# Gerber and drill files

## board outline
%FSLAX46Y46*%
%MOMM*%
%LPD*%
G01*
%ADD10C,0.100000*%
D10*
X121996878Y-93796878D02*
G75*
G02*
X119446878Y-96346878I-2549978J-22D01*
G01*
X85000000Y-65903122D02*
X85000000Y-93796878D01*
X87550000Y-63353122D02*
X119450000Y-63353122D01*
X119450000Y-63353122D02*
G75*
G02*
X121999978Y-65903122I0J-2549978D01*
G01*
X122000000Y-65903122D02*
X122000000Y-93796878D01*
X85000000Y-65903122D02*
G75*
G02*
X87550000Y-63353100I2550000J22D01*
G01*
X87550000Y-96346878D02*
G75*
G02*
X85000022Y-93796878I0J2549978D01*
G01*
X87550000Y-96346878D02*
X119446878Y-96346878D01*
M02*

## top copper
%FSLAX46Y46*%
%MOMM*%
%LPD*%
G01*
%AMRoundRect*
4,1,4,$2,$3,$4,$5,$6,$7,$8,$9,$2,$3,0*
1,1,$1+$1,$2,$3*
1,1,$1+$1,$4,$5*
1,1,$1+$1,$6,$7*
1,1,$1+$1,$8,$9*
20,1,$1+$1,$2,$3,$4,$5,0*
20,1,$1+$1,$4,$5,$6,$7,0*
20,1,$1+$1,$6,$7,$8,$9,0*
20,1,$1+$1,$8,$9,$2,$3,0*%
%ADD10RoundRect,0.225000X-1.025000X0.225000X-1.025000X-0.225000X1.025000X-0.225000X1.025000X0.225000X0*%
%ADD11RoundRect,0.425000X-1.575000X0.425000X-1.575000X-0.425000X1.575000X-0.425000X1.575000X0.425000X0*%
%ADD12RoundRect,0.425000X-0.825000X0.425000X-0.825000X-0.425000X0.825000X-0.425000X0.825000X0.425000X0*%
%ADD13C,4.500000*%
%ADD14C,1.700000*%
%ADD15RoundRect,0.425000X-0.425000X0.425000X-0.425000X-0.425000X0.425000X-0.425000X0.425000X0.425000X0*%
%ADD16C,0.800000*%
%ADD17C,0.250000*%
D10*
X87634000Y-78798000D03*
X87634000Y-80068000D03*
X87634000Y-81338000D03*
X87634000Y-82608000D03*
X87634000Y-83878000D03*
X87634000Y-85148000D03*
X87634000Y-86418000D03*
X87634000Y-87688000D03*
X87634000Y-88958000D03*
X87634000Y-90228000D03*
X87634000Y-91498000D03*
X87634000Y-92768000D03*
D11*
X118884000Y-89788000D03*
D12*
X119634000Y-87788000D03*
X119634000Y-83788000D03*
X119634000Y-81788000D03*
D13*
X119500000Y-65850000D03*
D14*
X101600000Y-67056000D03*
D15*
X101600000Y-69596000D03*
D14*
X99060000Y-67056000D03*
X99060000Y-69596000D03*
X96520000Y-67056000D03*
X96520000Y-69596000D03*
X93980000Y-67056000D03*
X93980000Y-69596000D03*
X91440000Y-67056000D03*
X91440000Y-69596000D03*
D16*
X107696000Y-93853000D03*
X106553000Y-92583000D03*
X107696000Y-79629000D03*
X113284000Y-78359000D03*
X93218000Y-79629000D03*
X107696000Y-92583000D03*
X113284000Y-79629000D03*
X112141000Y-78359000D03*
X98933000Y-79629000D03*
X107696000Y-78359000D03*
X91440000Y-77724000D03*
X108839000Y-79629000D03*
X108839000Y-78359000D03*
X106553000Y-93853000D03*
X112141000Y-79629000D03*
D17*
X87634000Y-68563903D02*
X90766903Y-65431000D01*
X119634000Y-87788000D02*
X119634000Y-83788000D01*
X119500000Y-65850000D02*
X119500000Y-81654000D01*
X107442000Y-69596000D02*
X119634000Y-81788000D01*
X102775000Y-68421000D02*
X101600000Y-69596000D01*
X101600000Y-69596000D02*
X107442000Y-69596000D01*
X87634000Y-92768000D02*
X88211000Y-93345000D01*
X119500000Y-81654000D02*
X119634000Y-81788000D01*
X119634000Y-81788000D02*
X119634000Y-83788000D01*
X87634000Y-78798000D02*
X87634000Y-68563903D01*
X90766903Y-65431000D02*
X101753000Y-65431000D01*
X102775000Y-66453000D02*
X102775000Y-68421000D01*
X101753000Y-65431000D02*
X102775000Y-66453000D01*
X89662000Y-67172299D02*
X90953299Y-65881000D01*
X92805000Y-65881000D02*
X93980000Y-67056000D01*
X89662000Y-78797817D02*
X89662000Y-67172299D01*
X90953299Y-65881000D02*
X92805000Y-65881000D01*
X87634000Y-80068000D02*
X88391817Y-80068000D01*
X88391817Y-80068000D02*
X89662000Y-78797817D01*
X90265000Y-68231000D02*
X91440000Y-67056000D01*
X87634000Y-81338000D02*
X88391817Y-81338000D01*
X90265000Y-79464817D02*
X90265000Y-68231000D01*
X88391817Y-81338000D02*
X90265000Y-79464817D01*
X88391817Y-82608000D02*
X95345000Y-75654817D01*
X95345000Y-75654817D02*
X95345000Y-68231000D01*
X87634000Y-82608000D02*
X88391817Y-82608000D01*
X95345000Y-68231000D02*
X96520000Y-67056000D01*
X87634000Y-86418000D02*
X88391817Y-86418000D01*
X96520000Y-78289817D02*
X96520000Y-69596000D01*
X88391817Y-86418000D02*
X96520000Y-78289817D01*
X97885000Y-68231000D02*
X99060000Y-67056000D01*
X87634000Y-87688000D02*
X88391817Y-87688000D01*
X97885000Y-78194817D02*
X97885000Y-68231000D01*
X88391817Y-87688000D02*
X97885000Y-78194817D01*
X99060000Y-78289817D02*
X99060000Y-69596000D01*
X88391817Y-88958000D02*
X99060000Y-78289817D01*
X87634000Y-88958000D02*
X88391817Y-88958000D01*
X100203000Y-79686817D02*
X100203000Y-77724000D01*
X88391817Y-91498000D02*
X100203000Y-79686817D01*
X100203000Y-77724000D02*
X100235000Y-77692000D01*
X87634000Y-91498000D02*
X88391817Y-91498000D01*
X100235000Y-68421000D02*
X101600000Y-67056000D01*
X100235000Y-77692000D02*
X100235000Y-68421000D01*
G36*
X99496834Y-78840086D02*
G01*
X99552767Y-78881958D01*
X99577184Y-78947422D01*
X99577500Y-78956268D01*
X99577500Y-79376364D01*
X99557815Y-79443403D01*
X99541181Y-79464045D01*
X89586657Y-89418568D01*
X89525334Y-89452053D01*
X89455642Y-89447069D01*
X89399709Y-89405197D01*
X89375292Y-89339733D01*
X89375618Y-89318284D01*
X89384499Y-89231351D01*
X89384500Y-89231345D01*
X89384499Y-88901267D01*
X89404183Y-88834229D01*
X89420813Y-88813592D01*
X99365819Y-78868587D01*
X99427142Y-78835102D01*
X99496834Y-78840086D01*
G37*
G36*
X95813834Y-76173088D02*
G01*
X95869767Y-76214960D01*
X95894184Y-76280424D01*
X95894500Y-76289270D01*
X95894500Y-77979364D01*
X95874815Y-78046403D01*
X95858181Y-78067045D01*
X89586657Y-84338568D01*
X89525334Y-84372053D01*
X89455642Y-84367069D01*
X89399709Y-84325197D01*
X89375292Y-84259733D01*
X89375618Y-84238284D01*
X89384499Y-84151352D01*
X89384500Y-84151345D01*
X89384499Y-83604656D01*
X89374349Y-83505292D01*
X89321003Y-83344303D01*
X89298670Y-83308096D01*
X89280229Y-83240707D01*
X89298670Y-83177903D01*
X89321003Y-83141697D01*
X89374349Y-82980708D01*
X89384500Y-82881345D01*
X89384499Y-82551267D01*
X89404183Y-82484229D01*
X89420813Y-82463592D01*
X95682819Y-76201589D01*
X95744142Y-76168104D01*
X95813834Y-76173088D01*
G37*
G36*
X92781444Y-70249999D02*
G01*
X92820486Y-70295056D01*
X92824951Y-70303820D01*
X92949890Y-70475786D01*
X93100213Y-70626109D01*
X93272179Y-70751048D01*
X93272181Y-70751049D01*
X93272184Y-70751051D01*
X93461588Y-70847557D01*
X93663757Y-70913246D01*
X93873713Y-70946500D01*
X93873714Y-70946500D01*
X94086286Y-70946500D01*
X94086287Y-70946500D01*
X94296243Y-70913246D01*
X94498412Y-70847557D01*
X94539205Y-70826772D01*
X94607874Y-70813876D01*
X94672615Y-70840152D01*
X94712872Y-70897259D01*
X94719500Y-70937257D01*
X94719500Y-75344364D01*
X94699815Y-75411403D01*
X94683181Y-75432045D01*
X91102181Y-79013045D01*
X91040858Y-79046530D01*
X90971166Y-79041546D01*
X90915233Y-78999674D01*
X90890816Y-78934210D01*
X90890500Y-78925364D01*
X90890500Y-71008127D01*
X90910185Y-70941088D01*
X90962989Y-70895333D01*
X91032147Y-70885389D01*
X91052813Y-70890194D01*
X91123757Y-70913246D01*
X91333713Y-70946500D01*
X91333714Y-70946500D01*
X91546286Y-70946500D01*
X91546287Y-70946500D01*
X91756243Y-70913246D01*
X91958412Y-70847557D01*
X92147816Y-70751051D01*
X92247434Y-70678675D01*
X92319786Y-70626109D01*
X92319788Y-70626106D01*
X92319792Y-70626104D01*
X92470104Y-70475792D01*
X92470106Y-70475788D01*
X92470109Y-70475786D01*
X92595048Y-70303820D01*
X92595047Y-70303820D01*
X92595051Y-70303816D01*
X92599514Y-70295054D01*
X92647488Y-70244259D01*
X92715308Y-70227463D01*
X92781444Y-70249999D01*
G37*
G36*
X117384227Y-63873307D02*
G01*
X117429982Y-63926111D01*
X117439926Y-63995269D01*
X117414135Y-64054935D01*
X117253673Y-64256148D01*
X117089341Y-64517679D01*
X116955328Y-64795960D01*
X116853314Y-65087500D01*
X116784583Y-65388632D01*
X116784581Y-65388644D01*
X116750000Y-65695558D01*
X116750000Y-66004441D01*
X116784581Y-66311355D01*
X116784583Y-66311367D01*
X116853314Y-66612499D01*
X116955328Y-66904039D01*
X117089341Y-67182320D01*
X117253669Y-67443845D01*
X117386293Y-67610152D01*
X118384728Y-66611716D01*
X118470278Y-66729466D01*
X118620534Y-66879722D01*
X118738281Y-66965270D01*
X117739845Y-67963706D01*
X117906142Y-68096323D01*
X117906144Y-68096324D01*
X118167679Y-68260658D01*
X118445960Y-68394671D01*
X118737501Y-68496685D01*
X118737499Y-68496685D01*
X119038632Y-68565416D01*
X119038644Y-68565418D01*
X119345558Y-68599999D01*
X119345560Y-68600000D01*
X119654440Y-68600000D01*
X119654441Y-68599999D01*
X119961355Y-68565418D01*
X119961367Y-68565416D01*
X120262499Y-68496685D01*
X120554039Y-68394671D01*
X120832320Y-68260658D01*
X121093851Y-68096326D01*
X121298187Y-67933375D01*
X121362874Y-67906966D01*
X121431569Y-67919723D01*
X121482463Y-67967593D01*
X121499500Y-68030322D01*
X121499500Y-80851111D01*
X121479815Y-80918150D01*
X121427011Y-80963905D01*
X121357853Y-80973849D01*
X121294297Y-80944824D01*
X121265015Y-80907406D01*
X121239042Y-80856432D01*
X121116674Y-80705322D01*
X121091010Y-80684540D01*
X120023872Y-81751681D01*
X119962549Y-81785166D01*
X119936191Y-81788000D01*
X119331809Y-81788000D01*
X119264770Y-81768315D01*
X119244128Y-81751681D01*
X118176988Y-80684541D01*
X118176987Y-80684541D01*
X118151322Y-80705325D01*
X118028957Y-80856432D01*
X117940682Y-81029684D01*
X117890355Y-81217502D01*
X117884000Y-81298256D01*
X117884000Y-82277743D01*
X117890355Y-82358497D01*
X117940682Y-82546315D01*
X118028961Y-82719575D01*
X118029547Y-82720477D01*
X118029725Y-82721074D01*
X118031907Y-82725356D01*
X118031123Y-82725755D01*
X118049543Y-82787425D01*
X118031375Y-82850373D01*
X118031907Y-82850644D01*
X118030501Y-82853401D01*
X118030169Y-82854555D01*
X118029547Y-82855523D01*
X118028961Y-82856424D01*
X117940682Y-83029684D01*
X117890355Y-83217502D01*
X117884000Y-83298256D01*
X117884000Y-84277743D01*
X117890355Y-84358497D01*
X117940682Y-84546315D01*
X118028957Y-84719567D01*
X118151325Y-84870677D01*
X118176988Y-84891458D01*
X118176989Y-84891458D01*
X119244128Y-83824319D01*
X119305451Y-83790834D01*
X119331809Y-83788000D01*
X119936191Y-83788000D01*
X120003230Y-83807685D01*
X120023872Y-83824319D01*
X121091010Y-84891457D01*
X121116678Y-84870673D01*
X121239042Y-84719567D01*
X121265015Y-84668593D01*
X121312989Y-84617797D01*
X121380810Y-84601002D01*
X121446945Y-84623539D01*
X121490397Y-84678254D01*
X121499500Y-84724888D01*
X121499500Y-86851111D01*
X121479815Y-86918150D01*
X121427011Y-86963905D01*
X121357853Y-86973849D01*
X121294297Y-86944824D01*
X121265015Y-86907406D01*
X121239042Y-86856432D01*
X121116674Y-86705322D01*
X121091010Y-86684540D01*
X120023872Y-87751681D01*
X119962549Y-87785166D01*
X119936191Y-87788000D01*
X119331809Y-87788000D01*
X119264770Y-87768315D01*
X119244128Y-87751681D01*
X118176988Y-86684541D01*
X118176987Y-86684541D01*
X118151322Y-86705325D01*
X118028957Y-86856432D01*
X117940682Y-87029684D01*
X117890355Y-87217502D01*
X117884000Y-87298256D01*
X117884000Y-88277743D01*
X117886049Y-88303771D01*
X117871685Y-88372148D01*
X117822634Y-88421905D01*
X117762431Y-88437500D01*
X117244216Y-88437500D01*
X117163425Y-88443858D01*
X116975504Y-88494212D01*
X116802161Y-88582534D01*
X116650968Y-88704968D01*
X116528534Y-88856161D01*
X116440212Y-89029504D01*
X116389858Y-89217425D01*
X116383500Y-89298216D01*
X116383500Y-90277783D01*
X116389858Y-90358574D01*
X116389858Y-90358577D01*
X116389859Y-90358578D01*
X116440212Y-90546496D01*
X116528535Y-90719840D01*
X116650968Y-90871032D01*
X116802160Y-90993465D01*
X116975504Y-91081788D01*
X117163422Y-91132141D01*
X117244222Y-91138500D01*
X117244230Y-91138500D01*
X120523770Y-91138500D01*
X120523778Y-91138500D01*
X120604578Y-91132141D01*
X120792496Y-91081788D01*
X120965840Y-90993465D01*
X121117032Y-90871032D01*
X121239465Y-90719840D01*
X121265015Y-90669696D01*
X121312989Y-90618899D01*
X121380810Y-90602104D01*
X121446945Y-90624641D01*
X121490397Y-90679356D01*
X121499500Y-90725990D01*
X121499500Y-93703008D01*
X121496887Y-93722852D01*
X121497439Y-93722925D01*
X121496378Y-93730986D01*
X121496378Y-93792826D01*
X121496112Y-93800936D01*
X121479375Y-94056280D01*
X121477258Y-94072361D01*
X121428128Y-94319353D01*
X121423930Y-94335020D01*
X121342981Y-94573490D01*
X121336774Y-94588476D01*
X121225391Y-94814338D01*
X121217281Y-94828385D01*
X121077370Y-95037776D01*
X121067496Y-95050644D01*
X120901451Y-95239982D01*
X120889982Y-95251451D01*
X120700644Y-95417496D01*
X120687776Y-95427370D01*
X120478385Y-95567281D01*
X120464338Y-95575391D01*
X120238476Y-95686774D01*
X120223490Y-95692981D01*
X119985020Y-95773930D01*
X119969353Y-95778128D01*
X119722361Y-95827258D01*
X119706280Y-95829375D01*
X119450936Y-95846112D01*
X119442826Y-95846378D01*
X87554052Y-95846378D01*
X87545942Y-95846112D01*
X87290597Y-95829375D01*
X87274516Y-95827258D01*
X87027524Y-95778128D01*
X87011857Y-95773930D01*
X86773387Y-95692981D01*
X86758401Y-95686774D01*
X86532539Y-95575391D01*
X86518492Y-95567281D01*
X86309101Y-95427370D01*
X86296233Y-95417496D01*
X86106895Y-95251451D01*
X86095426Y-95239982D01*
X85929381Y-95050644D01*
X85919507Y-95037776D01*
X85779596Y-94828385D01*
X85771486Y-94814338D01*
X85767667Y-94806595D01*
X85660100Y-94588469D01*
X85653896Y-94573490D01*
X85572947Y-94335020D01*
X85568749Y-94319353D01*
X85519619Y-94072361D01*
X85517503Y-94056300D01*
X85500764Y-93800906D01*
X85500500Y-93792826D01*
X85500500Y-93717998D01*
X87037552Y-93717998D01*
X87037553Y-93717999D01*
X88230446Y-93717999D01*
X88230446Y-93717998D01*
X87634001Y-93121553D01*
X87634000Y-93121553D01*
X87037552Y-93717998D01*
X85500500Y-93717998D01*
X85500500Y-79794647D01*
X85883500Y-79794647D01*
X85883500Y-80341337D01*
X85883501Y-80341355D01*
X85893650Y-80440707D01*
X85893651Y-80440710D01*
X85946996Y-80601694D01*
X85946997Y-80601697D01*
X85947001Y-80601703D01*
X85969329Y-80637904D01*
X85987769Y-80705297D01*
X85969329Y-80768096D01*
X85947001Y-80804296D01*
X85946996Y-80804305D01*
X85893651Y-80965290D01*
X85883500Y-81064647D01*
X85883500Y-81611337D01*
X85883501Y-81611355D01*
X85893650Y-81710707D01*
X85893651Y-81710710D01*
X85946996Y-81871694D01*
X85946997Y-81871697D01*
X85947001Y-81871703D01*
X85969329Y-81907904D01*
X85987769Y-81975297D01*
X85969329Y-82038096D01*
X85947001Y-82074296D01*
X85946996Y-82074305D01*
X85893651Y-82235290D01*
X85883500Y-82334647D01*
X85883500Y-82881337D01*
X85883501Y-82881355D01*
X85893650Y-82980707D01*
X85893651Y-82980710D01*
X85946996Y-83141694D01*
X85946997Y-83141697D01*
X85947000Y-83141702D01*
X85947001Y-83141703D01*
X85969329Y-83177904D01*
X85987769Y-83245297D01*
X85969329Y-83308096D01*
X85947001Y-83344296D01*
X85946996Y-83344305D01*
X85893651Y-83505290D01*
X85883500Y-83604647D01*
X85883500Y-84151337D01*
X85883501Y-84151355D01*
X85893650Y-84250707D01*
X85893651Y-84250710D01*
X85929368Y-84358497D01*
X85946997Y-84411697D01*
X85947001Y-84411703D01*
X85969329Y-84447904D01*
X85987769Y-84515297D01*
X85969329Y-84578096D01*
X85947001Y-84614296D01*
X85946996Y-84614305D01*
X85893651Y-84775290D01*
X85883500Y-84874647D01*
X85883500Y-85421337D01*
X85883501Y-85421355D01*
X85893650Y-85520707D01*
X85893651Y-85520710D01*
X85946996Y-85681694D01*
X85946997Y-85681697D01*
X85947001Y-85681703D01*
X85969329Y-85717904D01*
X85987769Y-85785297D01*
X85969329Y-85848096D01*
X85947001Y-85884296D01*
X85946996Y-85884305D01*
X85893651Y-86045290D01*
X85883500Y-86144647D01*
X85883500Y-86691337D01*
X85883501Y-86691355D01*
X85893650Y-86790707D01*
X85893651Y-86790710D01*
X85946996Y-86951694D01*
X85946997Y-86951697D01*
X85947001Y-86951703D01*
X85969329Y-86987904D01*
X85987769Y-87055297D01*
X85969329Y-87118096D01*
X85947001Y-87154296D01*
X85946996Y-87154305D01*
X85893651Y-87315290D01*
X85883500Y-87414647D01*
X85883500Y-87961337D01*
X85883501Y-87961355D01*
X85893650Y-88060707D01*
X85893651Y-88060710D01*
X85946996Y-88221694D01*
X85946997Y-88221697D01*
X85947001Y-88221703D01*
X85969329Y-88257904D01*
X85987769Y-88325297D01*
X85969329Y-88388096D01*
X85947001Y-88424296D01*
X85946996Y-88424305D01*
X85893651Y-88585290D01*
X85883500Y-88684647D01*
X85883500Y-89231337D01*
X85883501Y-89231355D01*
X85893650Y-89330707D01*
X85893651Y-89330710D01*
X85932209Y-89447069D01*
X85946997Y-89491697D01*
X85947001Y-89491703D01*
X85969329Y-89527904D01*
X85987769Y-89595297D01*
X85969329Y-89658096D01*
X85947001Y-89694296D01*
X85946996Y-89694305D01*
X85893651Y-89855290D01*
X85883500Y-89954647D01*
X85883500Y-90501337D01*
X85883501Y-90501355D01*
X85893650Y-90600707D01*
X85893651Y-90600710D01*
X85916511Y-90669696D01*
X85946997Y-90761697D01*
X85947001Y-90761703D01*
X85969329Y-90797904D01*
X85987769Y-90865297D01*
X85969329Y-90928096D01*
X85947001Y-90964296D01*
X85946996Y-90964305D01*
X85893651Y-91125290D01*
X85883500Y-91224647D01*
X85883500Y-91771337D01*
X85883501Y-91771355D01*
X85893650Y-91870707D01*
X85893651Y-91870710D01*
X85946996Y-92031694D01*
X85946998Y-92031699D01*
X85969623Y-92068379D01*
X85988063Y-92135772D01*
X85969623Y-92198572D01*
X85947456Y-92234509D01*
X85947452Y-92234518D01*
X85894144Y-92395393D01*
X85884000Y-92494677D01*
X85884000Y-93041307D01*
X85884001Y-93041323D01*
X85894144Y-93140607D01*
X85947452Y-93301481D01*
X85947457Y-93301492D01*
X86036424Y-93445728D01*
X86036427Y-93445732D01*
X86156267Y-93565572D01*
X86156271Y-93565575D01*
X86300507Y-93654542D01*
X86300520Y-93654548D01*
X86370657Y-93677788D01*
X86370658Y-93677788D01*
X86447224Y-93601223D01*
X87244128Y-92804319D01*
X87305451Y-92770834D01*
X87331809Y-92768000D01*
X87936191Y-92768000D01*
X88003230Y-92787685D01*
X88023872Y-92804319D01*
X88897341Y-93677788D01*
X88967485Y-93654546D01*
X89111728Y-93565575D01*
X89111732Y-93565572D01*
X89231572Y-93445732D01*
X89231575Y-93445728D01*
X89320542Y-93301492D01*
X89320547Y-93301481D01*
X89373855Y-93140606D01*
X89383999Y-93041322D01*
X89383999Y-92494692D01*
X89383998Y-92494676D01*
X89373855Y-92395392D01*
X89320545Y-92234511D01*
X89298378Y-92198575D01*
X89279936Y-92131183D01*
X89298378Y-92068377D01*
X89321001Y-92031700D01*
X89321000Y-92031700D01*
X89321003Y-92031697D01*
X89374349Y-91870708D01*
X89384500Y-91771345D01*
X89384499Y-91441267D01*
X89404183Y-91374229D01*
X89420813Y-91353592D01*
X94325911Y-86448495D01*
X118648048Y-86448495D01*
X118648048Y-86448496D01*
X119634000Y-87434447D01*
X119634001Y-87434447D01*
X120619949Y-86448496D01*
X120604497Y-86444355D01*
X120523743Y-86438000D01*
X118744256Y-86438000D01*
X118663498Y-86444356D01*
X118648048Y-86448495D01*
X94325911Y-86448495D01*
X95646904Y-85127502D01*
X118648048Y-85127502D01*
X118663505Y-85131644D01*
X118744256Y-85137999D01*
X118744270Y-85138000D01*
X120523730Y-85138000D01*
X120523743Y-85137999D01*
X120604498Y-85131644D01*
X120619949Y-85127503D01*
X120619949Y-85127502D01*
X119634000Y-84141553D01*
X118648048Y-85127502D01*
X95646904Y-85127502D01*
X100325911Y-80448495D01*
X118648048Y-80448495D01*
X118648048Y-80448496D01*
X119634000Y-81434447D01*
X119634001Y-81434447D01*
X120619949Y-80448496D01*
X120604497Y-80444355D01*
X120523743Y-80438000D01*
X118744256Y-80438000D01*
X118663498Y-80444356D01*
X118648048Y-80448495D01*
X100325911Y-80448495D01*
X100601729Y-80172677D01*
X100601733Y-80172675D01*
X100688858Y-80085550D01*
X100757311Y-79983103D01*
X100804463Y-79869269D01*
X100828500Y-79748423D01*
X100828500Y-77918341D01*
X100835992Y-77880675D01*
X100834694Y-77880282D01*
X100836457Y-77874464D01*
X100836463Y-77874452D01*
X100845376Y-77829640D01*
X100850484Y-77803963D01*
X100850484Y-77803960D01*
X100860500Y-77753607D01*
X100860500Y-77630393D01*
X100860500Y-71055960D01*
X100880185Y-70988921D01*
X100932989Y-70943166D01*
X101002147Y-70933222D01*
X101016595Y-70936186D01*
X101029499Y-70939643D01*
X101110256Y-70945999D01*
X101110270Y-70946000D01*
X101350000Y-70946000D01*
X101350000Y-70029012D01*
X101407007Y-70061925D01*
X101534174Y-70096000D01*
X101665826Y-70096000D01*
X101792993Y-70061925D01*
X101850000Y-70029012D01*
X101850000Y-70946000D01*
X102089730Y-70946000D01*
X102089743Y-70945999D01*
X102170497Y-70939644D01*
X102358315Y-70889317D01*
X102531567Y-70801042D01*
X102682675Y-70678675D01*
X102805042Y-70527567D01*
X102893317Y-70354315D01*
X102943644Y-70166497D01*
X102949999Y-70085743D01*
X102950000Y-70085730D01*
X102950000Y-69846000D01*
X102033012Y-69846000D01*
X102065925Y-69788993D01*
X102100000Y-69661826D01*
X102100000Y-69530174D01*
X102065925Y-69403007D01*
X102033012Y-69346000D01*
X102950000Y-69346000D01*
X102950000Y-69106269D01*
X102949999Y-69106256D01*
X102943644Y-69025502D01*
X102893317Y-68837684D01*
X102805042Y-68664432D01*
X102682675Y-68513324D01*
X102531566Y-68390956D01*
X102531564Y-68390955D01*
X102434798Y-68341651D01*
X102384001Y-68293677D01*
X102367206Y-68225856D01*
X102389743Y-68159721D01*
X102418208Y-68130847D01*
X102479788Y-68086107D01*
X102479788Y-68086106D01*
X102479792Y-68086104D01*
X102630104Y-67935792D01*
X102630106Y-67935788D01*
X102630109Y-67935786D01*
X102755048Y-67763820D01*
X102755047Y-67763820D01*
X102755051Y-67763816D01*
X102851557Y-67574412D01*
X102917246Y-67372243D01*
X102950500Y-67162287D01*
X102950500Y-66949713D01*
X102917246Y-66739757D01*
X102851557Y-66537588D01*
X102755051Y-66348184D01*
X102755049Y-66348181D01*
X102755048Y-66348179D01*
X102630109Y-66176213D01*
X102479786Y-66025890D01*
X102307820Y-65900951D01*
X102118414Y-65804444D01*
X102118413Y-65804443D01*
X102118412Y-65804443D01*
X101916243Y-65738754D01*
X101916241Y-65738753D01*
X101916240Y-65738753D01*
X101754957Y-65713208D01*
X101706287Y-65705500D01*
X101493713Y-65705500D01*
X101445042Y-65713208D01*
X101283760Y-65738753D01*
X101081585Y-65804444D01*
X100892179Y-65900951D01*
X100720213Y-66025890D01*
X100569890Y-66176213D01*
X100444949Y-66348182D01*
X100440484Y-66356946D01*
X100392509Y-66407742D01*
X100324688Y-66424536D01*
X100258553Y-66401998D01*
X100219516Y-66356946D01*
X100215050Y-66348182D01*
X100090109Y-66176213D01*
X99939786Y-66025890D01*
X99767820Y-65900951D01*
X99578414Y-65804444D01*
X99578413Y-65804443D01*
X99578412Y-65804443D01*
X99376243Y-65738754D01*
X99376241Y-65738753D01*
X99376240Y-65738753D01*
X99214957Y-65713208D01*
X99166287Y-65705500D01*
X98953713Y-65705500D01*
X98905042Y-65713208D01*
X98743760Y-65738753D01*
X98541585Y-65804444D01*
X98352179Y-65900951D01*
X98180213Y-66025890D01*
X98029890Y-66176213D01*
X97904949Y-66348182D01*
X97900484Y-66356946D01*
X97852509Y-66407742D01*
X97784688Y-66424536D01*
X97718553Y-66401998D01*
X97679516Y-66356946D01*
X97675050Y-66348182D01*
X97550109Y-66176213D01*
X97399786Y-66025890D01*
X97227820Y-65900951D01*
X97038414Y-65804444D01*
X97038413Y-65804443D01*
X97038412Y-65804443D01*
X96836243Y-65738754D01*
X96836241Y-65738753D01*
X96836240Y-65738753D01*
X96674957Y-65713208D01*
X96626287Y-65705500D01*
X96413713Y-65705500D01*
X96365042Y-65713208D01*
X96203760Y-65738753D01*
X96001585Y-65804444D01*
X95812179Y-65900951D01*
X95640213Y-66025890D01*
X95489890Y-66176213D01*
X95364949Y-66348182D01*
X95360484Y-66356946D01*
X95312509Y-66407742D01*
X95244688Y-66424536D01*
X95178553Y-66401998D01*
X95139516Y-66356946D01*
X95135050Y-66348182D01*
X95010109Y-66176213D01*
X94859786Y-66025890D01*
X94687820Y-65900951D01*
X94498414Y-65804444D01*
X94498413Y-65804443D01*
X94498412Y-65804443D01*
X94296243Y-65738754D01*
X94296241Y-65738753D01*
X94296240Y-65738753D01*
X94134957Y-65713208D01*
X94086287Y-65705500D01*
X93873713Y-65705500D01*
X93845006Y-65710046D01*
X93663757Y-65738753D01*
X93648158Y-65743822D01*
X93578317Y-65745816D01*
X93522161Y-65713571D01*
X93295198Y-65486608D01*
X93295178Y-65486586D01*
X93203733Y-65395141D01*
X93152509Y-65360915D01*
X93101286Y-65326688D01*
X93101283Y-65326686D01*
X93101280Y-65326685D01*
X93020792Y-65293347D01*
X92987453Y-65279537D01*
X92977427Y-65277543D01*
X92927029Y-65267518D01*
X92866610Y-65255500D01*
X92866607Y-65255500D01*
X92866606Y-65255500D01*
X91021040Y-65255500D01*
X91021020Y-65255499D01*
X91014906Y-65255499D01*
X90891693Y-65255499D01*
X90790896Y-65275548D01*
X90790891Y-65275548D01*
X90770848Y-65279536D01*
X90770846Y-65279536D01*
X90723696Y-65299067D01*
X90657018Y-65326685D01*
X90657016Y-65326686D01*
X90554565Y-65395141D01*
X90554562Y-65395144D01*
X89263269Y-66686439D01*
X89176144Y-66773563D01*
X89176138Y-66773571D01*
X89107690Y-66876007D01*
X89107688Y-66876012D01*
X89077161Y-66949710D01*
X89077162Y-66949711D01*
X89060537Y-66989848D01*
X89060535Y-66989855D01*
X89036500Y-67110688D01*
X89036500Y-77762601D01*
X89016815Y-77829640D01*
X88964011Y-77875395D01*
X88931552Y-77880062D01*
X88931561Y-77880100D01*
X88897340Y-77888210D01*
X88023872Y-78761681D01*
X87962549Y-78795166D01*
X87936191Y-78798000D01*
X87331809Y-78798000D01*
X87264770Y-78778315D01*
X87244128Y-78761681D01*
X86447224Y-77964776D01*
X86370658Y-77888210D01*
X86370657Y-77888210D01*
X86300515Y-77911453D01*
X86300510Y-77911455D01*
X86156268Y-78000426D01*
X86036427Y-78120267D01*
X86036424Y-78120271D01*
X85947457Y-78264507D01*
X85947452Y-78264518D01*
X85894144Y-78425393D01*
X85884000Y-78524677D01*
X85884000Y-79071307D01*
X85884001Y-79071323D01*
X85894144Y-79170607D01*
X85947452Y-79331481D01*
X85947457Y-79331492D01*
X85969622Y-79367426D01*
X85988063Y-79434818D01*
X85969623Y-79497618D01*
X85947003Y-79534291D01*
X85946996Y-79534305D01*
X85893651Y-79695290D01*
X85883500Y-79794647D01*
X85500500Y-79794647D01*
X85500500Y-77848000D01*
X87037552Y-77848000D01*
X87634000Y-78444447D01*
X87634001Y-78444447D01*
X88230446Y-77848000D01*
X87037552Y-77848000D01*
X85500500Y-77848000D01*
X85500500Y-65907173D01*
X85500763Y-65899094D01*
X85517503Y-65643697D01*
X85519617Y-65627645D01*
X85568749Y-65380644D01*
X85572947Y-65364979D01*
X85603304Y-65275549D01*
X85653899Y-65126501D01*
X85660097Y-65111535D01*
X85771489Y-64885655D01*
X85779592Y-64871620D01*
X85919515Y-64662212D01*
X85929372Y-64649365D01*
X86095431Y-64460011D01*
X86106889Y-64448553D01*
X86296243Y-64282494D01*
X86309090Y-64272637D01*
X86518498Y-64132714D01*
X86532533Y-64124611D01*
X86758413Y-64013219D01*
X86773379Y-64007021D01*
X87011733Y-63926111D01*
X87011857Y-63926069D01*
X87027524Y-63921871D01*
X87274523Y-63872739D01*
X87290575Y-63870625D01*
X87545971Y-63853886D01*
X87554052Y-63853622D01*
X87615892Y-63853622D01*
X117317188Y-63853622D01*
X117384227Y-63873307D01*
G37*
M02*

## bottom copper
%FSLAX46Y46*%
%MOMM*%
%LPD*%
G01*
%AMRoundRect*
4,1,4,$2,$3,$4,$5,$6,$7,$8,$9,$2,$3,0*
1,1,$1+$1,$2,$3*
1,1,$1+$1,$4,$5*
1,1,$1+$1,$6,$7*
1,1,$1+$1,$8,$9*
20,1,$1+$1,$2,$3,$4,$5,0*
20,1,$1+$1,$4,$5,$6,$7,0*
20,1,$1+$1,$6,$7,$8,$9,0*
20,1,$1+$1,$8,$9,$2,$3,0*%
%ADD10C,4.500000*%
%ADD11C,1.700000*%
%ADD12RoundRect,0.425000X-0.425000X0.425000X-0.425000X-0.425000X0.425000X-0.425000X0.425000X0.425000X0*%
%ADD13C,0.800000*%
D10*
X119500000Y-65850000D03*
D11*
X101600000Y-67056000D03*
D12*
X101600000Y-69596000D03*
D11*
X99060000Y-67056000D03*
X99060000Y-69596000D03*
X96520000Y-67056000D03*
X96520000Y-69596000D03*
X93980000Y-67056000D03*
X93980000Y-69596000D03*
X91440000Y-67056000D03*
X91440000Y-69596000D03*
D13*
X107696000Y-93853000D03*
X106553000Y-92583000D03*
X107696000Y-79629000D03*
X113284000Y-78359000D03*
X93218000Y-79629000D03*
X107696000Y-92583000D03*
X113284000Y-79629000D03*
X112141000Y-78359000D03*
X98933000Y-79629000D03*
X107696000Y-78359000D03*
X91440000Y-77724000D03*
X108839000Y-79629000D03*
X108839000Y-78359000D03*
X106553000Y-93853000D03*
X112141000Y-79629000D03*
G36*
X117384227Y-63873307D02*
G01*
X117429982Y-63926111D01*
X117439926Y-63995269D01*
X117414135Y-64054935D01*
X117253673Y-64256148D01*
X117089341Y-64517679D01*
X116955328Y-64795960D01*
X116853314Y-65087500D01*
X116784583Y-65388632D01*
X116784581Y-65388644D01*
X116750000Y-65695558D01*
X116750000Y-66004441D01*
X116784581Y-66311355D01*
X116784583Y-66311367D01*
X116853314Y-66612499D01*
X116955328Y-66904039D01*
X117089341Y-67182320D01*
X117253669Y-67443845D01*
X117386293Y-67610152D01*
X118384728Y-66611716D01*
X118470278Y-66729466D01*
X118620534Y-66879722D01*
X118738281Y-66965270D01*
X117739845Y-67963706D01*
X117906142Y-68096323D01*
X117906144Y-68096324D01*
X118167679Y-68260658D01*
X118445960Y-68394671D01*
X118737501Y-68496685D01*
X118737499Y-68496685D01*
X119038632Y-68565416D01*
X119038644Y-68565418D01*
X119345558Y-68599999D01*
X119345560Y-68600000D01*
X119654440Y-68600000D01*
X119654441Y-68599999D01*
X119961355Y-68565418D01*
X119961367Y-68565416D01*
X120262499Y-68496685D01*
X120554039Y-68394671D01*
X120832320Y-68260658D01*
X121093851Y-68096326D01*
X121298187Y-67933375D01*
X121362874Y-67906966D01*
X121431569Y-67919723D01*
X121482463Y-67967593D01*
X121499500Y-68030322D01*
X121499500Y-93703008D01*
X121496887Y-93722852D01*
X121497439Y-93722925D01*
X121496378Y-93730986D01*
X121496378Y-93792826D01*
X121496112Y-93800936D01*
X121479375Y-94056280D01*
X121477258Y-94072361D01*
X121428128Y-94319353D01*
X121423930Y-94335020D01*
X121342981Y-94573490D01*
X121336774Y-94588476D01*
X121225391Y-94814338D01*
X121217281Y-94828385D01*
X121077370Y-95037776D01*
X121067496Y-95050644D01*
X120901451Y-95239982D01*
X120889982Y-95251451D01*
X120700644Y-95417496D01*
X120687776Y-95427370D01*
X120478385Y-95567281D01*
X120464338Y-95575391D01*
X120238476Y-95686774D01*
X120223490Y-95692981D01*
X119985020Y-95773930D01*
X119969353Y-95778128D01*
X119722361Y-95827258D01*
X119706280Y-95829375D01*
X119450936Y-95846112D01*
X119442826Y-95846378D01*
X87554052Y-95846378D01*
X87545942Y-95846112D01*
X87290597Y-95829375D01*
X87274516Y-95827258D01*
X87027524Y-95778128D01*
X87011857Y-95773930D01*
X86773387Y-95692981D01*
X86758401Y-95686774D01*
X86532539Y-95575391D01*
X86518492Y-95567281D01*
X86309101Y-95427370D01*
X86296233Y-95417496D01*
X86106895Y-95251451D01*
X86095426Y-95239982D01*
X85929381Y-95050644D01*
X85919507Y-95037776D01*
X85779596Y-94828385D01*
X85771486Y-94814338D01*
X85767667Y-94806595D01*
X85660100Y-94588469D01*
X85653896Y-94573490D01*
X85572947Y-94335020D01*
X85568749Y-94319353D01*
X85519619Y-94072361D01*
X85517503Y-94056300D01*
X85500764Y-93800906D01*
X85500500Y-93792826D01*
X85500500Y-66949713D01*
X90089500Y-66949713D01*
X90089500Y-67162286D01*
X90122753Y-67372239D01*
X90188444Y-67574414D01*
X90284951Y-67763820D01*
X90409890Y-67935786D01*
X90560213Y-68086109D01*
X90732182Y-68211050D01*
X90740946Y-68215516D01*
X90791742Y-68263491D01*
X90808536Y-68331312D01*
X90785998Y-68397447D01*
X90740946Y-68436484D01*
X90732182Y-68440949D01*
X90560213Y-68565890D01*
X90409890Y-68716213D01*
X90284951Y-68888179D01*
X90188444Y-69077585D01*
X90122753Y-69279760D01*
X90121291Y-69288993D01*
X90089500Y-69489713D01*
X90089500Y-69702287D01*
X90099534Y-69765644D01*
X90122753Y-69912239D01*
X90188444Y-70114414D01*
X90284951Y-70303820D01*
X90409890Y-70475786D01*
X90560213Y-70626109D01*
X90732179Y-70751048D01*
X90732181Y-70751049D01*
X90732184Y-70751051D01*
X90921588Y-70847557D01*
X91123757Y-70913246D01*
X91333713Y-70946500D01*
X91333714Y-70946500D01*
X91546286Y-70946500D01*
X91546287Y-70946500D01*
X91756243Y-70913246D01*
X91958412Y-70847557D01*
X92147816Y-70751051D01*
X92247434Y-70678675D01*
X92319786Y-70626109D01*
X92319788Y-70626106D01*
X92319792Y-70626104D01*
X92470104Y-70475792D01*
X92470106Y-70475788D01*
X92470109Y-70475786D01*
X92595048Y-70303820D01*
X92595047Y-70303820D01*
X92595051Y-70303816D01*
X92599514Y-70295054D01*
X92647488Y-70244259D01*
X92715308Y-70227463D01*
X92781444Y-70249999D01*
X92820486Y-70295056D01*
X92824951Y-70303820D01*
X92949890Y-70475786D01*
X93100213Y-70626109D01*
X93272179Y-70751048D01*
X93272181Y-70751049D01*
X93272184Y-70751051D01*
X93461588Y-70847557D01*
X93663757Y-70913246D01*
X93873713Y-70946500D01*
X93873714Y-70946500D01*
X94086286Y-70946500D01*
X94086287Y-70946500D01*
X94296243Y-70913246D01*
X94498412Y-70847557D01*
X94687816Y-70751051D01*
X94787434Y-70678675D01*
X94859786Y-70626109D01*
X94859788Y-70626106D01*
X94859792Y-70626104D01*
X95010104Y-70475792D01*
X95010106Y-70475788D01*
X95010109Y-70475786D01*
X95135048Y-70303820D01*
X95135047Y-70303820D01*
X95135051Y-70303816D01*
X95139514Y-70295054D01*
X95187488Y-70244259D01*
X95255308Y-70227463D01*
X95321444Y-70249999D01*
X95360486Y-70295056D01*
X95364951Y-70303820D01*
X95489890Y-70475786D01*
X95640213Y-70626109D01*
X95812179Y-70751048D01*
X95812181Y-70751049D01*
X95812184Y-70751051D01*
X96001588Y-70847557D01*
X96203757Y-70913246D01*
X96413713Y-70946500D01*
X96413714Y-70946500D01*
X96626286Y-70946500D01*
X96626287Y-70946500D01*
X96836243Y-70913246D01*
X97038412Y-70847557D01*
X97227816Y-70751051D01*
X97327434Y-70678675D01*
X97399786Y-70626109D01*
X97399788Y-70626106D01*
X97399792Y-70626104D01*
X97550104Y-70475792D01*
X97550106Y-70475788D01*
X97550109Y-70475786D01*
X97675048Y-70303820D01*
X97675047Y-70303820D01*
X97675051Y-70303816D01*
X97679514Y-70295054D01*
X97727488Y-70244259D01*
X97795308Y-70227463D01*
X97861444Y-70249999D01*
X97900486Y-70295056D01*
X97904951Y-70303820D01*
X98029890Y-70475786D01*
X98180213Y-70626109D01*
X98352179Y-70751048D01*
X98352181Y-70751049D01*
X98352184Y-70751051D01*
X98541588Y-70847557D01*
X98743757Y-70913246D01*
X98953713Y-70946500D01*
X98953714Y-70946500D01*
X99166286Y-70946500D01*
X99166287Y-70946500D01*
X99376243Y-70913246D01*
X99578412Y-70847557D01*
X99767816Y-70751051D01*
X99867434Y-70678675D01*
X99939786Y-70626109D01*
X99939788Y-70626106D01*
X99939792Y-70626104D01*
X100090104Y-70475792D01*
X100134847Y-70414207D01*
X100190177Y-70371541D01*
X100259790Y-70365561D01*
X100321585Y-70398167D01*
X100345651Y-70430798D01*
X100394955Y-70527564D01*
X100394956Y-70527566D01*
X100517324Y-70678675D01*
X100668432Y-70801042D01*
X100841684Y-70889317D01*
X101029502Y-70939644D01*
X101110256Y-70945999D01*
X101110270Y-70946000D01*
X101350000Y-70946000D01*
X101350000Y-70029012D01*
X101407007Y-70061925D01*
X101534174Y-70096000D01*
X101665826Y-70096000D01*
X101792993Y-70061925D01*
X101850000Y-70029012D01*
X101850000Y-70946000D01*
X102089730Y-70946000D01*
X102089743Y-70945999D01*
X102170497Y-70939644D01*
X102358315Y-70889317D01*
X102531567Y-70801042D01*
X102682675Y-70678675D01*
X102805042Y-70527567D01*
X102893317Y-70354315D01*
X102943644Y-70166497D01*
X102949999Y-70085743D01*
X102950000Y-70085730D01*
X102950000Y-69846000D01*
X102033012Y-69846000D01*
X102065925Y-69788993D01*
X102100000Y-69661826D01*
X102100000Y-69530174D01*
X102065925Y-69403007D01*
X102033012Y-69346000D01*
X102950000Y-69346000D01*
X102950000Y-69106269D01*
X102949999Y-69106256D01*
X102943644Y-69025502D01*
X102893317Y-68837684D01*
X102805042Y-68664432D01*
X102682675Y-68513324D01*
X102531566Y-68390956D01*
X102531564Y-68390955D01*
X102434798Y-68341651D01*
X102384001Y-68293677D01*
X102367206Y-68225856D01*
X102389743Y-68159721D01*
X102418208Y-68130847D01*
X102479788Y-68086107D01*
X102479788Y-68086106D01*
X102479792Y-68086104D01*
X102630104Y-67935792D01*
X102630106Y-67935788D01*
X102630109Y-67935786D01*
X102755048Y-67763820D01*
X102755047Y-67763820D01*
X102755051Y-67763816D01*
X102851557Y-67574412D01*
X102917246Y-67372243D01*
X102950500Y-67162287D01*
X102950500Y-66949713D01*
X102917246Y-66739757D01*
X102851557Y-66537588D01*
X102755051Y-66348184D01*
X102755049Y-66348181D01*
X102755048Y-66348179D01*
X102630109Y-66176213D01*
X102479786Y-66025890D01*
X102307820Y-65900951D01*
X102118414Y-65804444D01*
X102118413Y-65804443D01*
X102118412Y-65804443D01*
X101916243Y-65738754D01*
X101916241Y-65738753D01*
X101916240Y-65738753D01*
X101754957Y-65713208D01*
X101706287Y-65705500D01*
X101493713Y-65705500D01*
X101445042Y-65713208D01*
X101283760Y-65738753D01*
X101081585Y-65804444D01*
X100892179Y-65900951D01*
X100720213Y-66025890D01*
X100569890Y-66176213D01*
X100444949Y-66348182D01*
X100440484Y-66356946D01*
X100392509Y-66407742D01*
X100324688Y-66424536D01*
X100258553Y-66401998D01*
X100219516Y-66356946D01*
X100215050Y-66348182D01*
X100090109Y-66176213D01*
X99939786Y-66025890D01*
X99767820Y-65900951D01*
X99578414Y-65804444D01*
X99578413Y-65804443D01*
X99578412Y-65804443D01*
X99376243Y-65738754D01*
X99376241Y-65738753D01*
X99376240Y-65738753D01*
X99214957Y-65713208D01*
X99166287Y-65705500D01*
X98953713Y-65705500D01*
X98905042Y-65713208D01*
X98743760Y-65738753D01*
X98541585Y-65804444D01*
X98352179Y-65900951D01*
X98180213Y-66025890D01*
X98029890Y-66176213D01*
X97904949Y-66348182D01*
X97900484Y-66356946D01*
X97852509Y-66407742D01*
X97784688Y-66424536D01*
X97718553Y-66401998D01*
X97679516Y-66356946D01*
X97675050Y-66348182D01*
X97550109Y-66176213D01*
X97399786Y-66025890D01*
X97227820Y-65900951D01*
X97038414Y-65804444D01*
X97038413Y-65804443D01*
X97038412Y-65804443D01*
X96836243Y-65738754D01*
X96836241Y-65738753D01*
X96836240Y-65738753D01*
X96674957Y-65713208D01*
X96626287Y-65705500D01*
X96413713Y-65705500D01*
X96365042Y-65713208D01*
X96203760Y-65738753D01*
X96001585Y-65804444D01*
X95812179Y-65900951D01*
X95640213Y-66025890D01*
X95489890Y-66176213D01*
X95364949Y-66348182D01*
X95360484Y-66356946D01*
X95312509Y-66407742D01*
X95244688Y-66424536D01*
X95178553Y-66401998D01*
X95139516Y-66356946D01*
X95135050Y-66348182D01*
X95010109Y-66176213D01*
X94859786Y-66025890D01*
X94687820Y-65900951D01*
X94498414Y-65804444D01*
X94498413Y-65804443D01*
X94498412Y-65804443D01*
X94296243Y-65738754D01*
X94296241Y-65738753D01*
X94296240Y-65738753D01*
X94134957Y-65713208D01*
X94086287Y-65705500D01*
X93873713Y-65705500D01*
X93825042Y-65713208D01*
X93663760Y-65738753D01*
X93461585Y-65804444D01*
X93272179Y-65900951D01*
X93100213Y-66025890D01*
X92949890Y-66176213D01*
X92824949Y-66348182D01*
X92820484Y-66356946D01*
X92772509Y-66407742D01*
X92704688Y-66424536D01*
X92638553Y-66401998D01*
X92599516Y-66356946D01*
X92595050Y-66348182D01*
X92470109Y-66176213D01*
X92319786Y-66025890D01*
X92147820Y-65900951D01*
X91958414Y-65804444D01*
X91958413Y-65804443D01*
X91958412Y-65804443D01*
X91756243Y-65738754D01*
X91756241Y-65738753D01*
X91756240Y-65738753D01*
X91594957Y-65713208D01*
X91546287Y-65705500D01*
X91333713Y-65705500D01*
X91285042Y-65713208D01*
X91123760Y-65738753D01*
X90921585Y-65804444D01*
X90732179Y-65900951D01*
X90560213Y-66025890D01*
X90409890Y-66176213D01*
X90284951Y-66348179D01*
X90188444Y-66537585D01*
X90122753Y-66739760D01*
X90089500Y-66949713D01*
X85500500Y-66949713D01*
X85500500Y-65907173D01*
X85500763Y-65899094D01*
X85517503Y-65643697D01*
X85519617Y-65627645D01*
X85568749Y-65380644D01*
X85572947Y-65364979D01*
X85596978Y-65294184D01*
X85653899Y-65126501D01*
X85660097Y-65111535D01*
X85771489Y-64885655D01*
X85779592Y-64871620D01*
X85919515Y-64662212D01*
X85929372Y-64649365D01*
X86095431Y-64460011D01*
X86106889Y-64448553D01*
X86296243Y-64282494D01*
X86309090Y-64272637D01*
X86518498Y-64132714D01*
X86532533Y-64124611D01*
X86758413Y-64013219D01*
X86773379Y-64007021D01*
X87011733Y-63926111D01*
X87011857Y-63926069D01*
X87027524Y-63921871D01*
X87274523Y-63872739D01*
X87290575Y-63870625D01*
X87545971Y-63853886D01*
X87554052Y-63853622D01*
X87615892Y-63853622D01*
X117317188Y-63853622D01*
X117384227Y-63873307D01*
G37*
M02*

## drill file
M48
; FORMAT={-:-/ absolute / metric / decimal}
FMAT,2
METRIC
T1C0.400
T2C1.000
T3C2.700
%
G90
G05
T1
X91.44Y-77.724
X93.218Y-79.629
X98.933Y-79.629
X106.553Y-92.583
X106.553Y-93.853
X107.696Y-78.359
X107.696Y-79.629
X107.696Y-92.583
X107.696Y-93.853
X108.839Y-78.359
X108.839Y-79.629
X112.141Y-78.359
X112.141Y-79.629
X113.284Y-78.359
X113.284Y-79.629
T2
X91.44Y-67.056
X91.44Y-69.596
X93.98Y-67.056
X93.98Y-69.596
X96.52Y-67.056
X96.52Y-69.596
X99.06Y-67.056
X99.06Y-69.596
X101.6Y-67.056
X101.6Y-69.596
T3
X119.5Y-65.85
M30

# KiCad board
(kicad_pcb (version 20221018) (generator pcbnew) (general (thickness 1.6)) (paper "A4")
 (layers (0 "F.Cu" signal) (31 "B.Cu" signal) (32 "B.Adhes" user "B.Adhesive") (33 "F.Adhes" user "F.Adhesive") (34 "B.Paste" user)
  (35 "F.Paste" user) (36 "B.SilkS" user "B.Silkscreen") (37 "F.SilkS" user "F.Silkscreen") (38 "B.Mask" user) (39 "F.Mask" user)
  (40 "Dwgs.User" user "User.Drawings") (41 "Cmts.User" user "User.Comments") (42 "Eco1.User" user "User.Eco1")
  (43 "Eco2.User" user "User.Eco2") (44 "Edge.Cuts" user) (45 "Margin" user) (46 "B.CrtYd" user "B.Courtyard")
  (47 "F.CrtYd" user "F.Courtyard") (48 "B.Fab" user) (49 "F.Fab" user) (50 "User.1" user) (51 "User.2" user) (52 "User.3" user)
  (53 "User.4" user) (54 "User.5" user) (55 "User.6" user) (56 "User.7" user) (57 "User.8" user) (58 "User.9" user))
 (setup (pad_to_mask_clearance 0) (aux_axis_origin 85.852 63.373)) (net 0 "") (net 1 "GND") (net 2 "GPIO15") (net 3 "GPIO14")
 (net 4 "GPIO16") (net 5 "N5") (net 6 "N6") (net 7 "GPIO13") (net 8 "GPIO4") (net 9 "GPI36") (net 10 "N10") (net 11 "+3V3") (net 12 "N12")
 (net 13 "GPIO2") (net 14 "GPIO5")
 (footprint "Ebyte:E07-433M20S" (layer "F.Cu") (at 119.634 94.788 90)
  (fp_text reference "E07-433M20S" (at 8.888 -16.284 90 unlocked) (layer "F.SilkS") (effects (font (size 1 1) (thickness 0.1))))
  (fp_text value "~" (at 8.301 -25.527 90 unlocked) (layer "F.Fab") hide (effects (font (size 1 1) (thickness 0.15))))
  (pad "1" smd roundrect (at 15.99 -32 270) (size 0.9 2.5) (layers "F.Cu" "F.Paste" "F.Mask") (roundrect_rratio 0.25) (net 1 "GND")
   (thermal_bridge_angle 45))
  (pad "2" smd roundrect (at 14.72 -32 270) (size 0.9 2.5) (layers "F.Cu" "F.Paste" "F.Mask") (roundrect_rratio 0.25) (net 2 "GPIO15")
   (thermal_bridge_angle 45))
  (pad "3" smd roundrect (at 13.45 -32 270) (size 0.9 2.5) (layers "F.Cu" "F.Paste" "F.Mask") (roundrect_rratio 0.25) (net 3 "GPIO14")
   (thermal_bridge_angle 45))
  (pad "4" smd roundrect (at 12.18 -32 270) (size 0.9 2.5) (layers "F.Cu" "F.Paste" "F.Mask") (roundrect_rratio 0.25) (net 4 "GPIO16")
   (thermal_bridge_angle 45))
  (pad "5" smd roundrect (at 10.91 -32 270) (size 0.9 2.5) (layers "F.Cu" "F.Paste" "F.Mask") (roundrect_rratio 0.25) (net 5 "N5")
   (thermal_bridge_angle 45))
  (pad "6" smd roundrect (at 9.64 -32 270) (size 0.9 2.5) (layers "F.Cu" "F.Paste" "F.Mask") (roundrect_rratio 0.25) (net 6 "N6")
   (thermal_bridge_angle 45))
  (pad "7" smd roundrect (at 8.37 -32 270) (size 0.9 2.5) (layers "F.Cu" "F.Paste" "F.Mask") (roundrect_rratio 0.25) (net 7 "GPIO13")
   (thermal_bridge_angle 45))
  (pad "8" smd roundrect (at 7.1 -32 270) (size 0.9 2.5) (layers "F.Cu" "F.Paste" "F.Mask") (roundrect_rratio 0.25) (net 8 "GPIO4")
   (thermal_bridge_angle 45))
  (pad "9" smd roundrect (at 5.83 -32 270) (size 0.9 2.5) (layers "F.Cu" "F.Paste" "F.Mask") (roundrect_rratio 0.25) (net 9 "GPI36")
   (thermal_bridge_angle 45))
  (pad "10" smd roundrect (at 4.56 -32 270) (size 0.9 2.5) (layers "F.Cu" "F.Paste" "F.Mask") (roundrect_rratio 0.25) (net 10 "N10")
   (thermal_bridge_angle 45))
  (pad "11" smd roundrect (at 3.29 -32 270) (size 0.9 2.5) (layers "F.Cu" "F.Paste" "F.Mask") (roundrect_rratio 0.25) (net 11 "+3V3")
   (thermal_bridge_angle 45))
  (pad "12" smd roundrect (at 2.02 -32 270) (size 0.9 2.5) (layers "F.Cu" "F.Paste" "F.Mask") (roundrect_rratio 0.25) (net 1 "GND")
   (thermal_bridge_angle 45))
  (pad "13" smd roundrect (at 5 -0.75 270) (size 1.7 4) (layers "F.Cu" "F.Paste" "F.Mask") (roundrect_rratio 0.25) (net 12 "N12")
   (thermal_bridge_angle 45))
  (pad "14" smd roundrect (at 7 0 270) (size 1.7 2.5) (layers "F.Cu" "F.Paste" "F.Mask") (roundrect_rratio 0.25) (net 1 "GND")
   (thermal_bridge_angle 45))
  (pad "15" smd roundrect (at 11 0 270) (size 1.7 2.5) (layers "F.Cu" "F.Paste" "F.Mask") (roundrect_rratio 0.25) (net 1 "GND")
   (thermal_bridge_angle 45))
  (pad "16" smd roundrect (at 13 0 270) (size 1.7 2.5) (layers "F.Cu" "F.Paste" "F.Mask") (roundrect_rratio 0.25) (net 1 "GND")
   (thermal_bridge_angle 45)))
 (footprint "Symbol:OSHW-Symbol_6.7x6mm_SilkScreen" (layer "F.Cu") (at 110.871 67.691)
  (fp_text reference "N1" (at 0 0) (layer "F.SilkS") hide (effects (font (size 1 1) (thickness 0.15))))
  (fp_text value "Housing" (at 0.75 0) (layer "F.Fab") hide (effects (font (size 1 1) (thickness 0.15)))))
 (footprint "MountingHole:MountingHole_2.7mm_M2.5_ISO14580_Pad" (layer "F.Cu") (at 119.5 65.85)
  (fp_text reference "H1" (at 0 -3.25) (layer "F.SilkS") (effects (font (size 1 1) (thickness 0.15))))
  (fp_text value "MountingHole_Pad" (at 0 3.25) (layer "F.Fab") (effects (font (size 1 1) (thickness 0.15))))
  (pad "1" thru_hole circle (at 0 0) (size 4.5 4.5) (drill 2.7) (layers "*.Cu" "*.Mask") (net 1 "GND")))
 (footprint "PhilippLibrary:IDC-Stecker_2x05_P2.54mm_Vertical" (layer "B.Cu") (at 91.44 67.056 -90)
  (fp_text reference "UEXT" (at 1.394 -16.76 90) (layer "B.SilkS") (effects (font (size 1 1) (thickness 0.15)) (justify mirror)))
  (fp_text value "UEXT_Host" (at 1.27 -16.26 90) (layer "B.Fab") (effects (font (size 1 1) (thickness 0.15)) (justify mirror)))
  (pad "1" thru_hole circle (at 0 -10.16 270) (size 1.7 1.7) (drill 1) (layers "*.Cu" "*.Mask") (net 11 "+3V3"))
  (pad "2" thru_hole roundrect (at 2.54 -10.16 270) (size 1.7 1.7) (drill 1) (layers "*.Cu" "*.Mask") (roundrect_rratio 0.25) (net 1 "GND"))
  (pad "3" thru_hole circle (at 0 -7.62 270) (size 1.7 1.7) (drill 1) (layers "*.Cu" "*.Mask") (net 8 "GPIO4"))
  (pad "4" thru_hole circle (at 2.54 -7.62 270) (size 1.7 1.7) (drill 1) (layers "*.Cu" "*.Mask") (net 9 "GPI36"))
  (pad "5" thru_hole circle (at 0 -5.08 270) (size 1.7 1.7) (drill 1) (layers "*.Cu" "*.Mask") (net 4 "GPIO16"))
  (pad "6" thru_hole circle (at 2.54 -5.08 270) (size 1.7 1.7) (drill 1) (layers "*.Cu" "*.Mask") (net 7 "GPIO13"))
  (pad "7" thru_hole circle (at 0 -2.54 270) (size 1.7 1.7) (drill 1) (layers "*.Cu" "*.Mask") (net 2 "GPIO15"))
  (pad "8" thru_hole circle (at 2.54 -2.54 270) (size 1.7 1.7) (drill 1) (layers "*.Cu" "*.Mask") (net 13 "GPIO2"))
  (pad "9" thru_hole circle (at 0 0 270) (size 1.7 1.7) (drill 1) (layers "*.Cu" "*.Mask") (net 3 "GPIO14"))
  (pad "10" thru_hole circle (at 2.54 0 270) (size 1.7 1.7) (drill 1) (layers "*.Cu" "*.Mask") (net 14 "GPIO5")))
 (gr_arc (start 121.996878 93.796878) (mid 121.25 95.6) (end 119.446878 96.346878) (stroke (width 0.1) (type default)) (layer "Edge.Cuts"))
 (gr_line (start 85 65.903122) (end 85 93.796878) (stroke (width 0.1) (type default)) (layer "Edge.Cuts"))
 (gr_line (start 87.55 63.353122) (end 119.45 63.353122) (stroke (width 0.1) (type default)) (layer "Edge.Cuts"))
 (gr_arc (start 119.45 63.353122) (mid 121.253122 64.1) (end 122 65.903122) (stroke (width 0.1) (type default)) (layer "Edge.Cuts"))
 (gr_line (start 122 65.903122) (end 122 93.796878) (stroke (width 0.1) (type default)) (layer "Edge.Cuts"))
 (gr_arc (start 85 65.903122) (mid 85.746878 64.1) (end 87.55 63.353122) (stroke (width 0.1) (type default)) (layer "Edge.Cuts"))
 (gr_arc (start 87.55 96.346878) (mid 85.746878 95.6) (end 85 93.796878) (stroke (width 0.1) (type default)) (layer "Edge.Cuts"))
 (gr_line (start 87.55 96.346878) (end 119.446878 96.346878) (stroke (width 0.1) (type default)) (layer "Edge.Cuts"))
 (segment (start 87.634 68.563903) (end 90.766903 65.431) (width 0.25) (layer "F.Cu") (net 1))
 (segment (start 119.634 87.788) (end 119.634 83.788) (width 0.25) (layer "F.Cu") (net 1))
 (segment (start 119.5 65.85) (end 119.5 81.654) (width 0.25) (layer "F.Cu") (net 1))
 (segment (start 107.442 69.596) (end 119.634 81.788) (width 0.25) (layer "F.Cu") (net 1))
 (segment (start 102.775 68.421) (end 101.6 69.596) (width 0.25) (layer "F.Cu") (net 1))
 (segment (start 101.6 69.596) (end 107.442 69.596) (width 0.25) (layer "F.Cu") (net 1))
 (segment (start 87.634 92.768) (end 88.211 93.345) (width 0.25) (layer "F.Cu") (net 1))
 (segment (start 119.5 81.654) (end 119.634 81.788) (width 0.25) (layer "F.Cu") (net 1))
 (segment (start 119.634 81.788) (end 119.634 83.788) (width 0.25) (layer "F.Cu") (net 1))
 (segment (start 87.634 78.798) (end 87.634 68.563903) (width 0.25) (layer "F.Cu") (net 1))
 (segment (start 90.766903 65.431) (end 101.753 65.431) (width 0.25) (layer "F.Cu") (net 1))
 (segment (start 102.775 66.453) (end 102.775 68.421) (width 0.25) (layer "F.Cu") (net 1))
 (segment (start 101.753 65.431) (end 102.775 66.453) (width 0.25) (layer "F.Cu") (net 1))
 (via (at 107.696 93.853) (size 0.8) (drill 0.4) (layers "F.Cu" "B.Cu") (free) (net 1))
 (via (at 106.553 92.583) (size 0.8) (drill 0.4) (layers "F.Cu" "B.Cu") (free) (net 1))
 (via (at 107.696 79.629) (size 0.8) (drill 0.4) (layers "F.Cu" "B.Cu") (free) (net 1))
 (via (at 113.284 78.359) (size 0.8) (drill 0.4) (layers "F.Cu" "B.Cu") (free) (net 1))
 (via (at 93.218 79.629) (size 0.8) (drill 0.4) (layers "F.Cu" "B.Cu") (free) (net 1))
 (via (at 107.696 92.583) (size 0.8) (drill 0.4) (layers "F.Cu" "B.Cu") (free) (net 1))
 (via (at 113.284 79.629) (size 0.8) (drill 0.4) (layers "F.Cu" "B.Cu") (free) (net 1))
 (via (at 112.141 78.359) (size 0.8) (drill 0.4) (layers "F.Cu" "B.Cu") (free) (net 1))
 (via (at 98.933 79.629) (size 0.8) (drill 0.4) (layers "F.Cu" "B.Cu") (free) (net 1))
 (via (at 107.696 78.359) (size 0.8) (drill 0.4) (layers "F.Cu" "B.Cu") (free) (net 1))
 (via (at 91.44 77.724) (size 0.8) (drill 0.4) (layers "F.Cu" "B.Cu") (free) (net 1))
 (via (at 108.839 79.629) (size 0.8) (drill 0.4) (layers "F.Cu" "B.Cu") (free) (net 1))
 (via (at 108.839 78.359) (size 0.8) (drill 0.4) (layers "F.Cu" "B.Cu") (free) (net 1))
 (via (at 106.553 93.853) (size 0.8) (drill 0.4) (layers "F.Cu" "B.Cu") (free) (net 1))
 (via (at 112.141 79.629) (size 0.8) (drill 0.4) (layers "F.Cu" "B.Cu") (free) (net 1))
 (segment (start 89.662 67.172299) (end 90.953299 65.881) (width 0.25) (layer "F.Cu") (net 2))
 (segment (start 92.805 65.881) (end 93.98 67.056) (width 0.25) (layer "F.Cu") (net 2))
 (segment (start 89.662 78.797817) (end 89.662 67.172299) (width 0.25) (layer "F.Cu") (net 2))
 (segment (start 90.953299 65.881) (end 92.805 65.881) (width 0.25) (layer "F.Cu") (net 2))
 (segment (start 87.634 80.068) (end 88.391817 80.068) (width 0.25) (layer "F.Cu") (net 2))
 (segment (start 88.391817 80.068) (end 89.662 78.797817) (width 0.25) (layer "F.Cu") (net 2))
 (segment (start 90.265 68.231) (end 91.44 67.056) (width 0.25) (layer "F.Cu") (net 3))
 (segment (start 87.634 81.338) (end 88.391817 81.338) (width 0.25) (layer "F.Cu") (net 3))
 (segment (start 90.265 79.464817) (end 90.265 68.231) (width 0.25) (layer "F.Cu") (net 3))
 (segment (start 88.391817 81.338) (end 90.265 79.464817) (width 0.25) (layer "F.Cu") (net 3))
 (segment (start 88.391817 82.608) (end 95.345 75.654817) (width 0.25) (layer "F.Cu") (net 4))
 (segment (start 95.345 75.654817) (end 95.345 68.231) (width 0.25) (layer "F.Cu") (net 4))
 (segment (start 87.634 82.608) (end 88.391817 82.608) (width 0.25) (layer "F.Cu") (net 4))
 (segment (start 95.345 68.231) (end 96.52 67.056) (width 0.25) (layer "F.Cu") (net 4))
 (segment (start 87.634 86.418) (end 88.391817 86.418) (width 0.25) (layer "F.Cu") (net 7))
 (segment (start 96.52 78.289817) (end 96.52 69.596) (width 0.25) (layer "F.Cu") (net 7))
 (segment (start 88.391817 86.418) (end 96.52 78.289817) (width 0.25) (layer "F.Cu") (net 7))
 (segment (start 97.885 68.231) (end 99.06 67.056) (width 0.25) (layer "F.Cu") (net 8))
 (segment (start 87.634 87.688) (end 88.391817 87.688) (width 0.25) (layer "F.Cu") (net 8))
 (segment (start 97.885 78.194817) (end 97.885 68.231) (width 0.25) (layer "F.Cu") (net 8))
 (segment (start 88.391817 87.688) (end 97.885 78.194817) (width 0.25) (layer "F.Cu") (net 8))
 (segment (start 99.06 78.289817) (end 99.06 69.596) (width 0.25) (layer "F.Cu") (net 9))
 (segment (start 88.391817 88.958) (end 99.06 78.289817) (width 0.25) (layer "F.Cu") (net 9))
 (segment (start 87.634 88.958) (end 88.391817 88.958) (width 0.25) (layer "F.Cu") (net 9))
 (segment (start 100.203 79.686817) (end 100.203 77.724) (width 0.25) (layer "F.Cu") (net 11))
 (segment (start 88.391817 91.498) (end 100.203 79.686817) (width 0.25) (layer "F.Cu") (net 11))
 (segment (start 100.203 77.724) (end 100.235 77.692) (width 0.25) (layer "F.Cu") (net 11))
 (segment (start 87.634 91.498) (end 88.391817 91.498) (width 0.25) (layer "F.Cu") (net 11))
 (segment (start 100.235 68.421) (end 101.6 67.056) (width 0.25) (layer "F.Cu") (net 11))
 (segment (start 100.235 77.692) (end 100.235 68.421) (width 0.25) (layer "F.Cu") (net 11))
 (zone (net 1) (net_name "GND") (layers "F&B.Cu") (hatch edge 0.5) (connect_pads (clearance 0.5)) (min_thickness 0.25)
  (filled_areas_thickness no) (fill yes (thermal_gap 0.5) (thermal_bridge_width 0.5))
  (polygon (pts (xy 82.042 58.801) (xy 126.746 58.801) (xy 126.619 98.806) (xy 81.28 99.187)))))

